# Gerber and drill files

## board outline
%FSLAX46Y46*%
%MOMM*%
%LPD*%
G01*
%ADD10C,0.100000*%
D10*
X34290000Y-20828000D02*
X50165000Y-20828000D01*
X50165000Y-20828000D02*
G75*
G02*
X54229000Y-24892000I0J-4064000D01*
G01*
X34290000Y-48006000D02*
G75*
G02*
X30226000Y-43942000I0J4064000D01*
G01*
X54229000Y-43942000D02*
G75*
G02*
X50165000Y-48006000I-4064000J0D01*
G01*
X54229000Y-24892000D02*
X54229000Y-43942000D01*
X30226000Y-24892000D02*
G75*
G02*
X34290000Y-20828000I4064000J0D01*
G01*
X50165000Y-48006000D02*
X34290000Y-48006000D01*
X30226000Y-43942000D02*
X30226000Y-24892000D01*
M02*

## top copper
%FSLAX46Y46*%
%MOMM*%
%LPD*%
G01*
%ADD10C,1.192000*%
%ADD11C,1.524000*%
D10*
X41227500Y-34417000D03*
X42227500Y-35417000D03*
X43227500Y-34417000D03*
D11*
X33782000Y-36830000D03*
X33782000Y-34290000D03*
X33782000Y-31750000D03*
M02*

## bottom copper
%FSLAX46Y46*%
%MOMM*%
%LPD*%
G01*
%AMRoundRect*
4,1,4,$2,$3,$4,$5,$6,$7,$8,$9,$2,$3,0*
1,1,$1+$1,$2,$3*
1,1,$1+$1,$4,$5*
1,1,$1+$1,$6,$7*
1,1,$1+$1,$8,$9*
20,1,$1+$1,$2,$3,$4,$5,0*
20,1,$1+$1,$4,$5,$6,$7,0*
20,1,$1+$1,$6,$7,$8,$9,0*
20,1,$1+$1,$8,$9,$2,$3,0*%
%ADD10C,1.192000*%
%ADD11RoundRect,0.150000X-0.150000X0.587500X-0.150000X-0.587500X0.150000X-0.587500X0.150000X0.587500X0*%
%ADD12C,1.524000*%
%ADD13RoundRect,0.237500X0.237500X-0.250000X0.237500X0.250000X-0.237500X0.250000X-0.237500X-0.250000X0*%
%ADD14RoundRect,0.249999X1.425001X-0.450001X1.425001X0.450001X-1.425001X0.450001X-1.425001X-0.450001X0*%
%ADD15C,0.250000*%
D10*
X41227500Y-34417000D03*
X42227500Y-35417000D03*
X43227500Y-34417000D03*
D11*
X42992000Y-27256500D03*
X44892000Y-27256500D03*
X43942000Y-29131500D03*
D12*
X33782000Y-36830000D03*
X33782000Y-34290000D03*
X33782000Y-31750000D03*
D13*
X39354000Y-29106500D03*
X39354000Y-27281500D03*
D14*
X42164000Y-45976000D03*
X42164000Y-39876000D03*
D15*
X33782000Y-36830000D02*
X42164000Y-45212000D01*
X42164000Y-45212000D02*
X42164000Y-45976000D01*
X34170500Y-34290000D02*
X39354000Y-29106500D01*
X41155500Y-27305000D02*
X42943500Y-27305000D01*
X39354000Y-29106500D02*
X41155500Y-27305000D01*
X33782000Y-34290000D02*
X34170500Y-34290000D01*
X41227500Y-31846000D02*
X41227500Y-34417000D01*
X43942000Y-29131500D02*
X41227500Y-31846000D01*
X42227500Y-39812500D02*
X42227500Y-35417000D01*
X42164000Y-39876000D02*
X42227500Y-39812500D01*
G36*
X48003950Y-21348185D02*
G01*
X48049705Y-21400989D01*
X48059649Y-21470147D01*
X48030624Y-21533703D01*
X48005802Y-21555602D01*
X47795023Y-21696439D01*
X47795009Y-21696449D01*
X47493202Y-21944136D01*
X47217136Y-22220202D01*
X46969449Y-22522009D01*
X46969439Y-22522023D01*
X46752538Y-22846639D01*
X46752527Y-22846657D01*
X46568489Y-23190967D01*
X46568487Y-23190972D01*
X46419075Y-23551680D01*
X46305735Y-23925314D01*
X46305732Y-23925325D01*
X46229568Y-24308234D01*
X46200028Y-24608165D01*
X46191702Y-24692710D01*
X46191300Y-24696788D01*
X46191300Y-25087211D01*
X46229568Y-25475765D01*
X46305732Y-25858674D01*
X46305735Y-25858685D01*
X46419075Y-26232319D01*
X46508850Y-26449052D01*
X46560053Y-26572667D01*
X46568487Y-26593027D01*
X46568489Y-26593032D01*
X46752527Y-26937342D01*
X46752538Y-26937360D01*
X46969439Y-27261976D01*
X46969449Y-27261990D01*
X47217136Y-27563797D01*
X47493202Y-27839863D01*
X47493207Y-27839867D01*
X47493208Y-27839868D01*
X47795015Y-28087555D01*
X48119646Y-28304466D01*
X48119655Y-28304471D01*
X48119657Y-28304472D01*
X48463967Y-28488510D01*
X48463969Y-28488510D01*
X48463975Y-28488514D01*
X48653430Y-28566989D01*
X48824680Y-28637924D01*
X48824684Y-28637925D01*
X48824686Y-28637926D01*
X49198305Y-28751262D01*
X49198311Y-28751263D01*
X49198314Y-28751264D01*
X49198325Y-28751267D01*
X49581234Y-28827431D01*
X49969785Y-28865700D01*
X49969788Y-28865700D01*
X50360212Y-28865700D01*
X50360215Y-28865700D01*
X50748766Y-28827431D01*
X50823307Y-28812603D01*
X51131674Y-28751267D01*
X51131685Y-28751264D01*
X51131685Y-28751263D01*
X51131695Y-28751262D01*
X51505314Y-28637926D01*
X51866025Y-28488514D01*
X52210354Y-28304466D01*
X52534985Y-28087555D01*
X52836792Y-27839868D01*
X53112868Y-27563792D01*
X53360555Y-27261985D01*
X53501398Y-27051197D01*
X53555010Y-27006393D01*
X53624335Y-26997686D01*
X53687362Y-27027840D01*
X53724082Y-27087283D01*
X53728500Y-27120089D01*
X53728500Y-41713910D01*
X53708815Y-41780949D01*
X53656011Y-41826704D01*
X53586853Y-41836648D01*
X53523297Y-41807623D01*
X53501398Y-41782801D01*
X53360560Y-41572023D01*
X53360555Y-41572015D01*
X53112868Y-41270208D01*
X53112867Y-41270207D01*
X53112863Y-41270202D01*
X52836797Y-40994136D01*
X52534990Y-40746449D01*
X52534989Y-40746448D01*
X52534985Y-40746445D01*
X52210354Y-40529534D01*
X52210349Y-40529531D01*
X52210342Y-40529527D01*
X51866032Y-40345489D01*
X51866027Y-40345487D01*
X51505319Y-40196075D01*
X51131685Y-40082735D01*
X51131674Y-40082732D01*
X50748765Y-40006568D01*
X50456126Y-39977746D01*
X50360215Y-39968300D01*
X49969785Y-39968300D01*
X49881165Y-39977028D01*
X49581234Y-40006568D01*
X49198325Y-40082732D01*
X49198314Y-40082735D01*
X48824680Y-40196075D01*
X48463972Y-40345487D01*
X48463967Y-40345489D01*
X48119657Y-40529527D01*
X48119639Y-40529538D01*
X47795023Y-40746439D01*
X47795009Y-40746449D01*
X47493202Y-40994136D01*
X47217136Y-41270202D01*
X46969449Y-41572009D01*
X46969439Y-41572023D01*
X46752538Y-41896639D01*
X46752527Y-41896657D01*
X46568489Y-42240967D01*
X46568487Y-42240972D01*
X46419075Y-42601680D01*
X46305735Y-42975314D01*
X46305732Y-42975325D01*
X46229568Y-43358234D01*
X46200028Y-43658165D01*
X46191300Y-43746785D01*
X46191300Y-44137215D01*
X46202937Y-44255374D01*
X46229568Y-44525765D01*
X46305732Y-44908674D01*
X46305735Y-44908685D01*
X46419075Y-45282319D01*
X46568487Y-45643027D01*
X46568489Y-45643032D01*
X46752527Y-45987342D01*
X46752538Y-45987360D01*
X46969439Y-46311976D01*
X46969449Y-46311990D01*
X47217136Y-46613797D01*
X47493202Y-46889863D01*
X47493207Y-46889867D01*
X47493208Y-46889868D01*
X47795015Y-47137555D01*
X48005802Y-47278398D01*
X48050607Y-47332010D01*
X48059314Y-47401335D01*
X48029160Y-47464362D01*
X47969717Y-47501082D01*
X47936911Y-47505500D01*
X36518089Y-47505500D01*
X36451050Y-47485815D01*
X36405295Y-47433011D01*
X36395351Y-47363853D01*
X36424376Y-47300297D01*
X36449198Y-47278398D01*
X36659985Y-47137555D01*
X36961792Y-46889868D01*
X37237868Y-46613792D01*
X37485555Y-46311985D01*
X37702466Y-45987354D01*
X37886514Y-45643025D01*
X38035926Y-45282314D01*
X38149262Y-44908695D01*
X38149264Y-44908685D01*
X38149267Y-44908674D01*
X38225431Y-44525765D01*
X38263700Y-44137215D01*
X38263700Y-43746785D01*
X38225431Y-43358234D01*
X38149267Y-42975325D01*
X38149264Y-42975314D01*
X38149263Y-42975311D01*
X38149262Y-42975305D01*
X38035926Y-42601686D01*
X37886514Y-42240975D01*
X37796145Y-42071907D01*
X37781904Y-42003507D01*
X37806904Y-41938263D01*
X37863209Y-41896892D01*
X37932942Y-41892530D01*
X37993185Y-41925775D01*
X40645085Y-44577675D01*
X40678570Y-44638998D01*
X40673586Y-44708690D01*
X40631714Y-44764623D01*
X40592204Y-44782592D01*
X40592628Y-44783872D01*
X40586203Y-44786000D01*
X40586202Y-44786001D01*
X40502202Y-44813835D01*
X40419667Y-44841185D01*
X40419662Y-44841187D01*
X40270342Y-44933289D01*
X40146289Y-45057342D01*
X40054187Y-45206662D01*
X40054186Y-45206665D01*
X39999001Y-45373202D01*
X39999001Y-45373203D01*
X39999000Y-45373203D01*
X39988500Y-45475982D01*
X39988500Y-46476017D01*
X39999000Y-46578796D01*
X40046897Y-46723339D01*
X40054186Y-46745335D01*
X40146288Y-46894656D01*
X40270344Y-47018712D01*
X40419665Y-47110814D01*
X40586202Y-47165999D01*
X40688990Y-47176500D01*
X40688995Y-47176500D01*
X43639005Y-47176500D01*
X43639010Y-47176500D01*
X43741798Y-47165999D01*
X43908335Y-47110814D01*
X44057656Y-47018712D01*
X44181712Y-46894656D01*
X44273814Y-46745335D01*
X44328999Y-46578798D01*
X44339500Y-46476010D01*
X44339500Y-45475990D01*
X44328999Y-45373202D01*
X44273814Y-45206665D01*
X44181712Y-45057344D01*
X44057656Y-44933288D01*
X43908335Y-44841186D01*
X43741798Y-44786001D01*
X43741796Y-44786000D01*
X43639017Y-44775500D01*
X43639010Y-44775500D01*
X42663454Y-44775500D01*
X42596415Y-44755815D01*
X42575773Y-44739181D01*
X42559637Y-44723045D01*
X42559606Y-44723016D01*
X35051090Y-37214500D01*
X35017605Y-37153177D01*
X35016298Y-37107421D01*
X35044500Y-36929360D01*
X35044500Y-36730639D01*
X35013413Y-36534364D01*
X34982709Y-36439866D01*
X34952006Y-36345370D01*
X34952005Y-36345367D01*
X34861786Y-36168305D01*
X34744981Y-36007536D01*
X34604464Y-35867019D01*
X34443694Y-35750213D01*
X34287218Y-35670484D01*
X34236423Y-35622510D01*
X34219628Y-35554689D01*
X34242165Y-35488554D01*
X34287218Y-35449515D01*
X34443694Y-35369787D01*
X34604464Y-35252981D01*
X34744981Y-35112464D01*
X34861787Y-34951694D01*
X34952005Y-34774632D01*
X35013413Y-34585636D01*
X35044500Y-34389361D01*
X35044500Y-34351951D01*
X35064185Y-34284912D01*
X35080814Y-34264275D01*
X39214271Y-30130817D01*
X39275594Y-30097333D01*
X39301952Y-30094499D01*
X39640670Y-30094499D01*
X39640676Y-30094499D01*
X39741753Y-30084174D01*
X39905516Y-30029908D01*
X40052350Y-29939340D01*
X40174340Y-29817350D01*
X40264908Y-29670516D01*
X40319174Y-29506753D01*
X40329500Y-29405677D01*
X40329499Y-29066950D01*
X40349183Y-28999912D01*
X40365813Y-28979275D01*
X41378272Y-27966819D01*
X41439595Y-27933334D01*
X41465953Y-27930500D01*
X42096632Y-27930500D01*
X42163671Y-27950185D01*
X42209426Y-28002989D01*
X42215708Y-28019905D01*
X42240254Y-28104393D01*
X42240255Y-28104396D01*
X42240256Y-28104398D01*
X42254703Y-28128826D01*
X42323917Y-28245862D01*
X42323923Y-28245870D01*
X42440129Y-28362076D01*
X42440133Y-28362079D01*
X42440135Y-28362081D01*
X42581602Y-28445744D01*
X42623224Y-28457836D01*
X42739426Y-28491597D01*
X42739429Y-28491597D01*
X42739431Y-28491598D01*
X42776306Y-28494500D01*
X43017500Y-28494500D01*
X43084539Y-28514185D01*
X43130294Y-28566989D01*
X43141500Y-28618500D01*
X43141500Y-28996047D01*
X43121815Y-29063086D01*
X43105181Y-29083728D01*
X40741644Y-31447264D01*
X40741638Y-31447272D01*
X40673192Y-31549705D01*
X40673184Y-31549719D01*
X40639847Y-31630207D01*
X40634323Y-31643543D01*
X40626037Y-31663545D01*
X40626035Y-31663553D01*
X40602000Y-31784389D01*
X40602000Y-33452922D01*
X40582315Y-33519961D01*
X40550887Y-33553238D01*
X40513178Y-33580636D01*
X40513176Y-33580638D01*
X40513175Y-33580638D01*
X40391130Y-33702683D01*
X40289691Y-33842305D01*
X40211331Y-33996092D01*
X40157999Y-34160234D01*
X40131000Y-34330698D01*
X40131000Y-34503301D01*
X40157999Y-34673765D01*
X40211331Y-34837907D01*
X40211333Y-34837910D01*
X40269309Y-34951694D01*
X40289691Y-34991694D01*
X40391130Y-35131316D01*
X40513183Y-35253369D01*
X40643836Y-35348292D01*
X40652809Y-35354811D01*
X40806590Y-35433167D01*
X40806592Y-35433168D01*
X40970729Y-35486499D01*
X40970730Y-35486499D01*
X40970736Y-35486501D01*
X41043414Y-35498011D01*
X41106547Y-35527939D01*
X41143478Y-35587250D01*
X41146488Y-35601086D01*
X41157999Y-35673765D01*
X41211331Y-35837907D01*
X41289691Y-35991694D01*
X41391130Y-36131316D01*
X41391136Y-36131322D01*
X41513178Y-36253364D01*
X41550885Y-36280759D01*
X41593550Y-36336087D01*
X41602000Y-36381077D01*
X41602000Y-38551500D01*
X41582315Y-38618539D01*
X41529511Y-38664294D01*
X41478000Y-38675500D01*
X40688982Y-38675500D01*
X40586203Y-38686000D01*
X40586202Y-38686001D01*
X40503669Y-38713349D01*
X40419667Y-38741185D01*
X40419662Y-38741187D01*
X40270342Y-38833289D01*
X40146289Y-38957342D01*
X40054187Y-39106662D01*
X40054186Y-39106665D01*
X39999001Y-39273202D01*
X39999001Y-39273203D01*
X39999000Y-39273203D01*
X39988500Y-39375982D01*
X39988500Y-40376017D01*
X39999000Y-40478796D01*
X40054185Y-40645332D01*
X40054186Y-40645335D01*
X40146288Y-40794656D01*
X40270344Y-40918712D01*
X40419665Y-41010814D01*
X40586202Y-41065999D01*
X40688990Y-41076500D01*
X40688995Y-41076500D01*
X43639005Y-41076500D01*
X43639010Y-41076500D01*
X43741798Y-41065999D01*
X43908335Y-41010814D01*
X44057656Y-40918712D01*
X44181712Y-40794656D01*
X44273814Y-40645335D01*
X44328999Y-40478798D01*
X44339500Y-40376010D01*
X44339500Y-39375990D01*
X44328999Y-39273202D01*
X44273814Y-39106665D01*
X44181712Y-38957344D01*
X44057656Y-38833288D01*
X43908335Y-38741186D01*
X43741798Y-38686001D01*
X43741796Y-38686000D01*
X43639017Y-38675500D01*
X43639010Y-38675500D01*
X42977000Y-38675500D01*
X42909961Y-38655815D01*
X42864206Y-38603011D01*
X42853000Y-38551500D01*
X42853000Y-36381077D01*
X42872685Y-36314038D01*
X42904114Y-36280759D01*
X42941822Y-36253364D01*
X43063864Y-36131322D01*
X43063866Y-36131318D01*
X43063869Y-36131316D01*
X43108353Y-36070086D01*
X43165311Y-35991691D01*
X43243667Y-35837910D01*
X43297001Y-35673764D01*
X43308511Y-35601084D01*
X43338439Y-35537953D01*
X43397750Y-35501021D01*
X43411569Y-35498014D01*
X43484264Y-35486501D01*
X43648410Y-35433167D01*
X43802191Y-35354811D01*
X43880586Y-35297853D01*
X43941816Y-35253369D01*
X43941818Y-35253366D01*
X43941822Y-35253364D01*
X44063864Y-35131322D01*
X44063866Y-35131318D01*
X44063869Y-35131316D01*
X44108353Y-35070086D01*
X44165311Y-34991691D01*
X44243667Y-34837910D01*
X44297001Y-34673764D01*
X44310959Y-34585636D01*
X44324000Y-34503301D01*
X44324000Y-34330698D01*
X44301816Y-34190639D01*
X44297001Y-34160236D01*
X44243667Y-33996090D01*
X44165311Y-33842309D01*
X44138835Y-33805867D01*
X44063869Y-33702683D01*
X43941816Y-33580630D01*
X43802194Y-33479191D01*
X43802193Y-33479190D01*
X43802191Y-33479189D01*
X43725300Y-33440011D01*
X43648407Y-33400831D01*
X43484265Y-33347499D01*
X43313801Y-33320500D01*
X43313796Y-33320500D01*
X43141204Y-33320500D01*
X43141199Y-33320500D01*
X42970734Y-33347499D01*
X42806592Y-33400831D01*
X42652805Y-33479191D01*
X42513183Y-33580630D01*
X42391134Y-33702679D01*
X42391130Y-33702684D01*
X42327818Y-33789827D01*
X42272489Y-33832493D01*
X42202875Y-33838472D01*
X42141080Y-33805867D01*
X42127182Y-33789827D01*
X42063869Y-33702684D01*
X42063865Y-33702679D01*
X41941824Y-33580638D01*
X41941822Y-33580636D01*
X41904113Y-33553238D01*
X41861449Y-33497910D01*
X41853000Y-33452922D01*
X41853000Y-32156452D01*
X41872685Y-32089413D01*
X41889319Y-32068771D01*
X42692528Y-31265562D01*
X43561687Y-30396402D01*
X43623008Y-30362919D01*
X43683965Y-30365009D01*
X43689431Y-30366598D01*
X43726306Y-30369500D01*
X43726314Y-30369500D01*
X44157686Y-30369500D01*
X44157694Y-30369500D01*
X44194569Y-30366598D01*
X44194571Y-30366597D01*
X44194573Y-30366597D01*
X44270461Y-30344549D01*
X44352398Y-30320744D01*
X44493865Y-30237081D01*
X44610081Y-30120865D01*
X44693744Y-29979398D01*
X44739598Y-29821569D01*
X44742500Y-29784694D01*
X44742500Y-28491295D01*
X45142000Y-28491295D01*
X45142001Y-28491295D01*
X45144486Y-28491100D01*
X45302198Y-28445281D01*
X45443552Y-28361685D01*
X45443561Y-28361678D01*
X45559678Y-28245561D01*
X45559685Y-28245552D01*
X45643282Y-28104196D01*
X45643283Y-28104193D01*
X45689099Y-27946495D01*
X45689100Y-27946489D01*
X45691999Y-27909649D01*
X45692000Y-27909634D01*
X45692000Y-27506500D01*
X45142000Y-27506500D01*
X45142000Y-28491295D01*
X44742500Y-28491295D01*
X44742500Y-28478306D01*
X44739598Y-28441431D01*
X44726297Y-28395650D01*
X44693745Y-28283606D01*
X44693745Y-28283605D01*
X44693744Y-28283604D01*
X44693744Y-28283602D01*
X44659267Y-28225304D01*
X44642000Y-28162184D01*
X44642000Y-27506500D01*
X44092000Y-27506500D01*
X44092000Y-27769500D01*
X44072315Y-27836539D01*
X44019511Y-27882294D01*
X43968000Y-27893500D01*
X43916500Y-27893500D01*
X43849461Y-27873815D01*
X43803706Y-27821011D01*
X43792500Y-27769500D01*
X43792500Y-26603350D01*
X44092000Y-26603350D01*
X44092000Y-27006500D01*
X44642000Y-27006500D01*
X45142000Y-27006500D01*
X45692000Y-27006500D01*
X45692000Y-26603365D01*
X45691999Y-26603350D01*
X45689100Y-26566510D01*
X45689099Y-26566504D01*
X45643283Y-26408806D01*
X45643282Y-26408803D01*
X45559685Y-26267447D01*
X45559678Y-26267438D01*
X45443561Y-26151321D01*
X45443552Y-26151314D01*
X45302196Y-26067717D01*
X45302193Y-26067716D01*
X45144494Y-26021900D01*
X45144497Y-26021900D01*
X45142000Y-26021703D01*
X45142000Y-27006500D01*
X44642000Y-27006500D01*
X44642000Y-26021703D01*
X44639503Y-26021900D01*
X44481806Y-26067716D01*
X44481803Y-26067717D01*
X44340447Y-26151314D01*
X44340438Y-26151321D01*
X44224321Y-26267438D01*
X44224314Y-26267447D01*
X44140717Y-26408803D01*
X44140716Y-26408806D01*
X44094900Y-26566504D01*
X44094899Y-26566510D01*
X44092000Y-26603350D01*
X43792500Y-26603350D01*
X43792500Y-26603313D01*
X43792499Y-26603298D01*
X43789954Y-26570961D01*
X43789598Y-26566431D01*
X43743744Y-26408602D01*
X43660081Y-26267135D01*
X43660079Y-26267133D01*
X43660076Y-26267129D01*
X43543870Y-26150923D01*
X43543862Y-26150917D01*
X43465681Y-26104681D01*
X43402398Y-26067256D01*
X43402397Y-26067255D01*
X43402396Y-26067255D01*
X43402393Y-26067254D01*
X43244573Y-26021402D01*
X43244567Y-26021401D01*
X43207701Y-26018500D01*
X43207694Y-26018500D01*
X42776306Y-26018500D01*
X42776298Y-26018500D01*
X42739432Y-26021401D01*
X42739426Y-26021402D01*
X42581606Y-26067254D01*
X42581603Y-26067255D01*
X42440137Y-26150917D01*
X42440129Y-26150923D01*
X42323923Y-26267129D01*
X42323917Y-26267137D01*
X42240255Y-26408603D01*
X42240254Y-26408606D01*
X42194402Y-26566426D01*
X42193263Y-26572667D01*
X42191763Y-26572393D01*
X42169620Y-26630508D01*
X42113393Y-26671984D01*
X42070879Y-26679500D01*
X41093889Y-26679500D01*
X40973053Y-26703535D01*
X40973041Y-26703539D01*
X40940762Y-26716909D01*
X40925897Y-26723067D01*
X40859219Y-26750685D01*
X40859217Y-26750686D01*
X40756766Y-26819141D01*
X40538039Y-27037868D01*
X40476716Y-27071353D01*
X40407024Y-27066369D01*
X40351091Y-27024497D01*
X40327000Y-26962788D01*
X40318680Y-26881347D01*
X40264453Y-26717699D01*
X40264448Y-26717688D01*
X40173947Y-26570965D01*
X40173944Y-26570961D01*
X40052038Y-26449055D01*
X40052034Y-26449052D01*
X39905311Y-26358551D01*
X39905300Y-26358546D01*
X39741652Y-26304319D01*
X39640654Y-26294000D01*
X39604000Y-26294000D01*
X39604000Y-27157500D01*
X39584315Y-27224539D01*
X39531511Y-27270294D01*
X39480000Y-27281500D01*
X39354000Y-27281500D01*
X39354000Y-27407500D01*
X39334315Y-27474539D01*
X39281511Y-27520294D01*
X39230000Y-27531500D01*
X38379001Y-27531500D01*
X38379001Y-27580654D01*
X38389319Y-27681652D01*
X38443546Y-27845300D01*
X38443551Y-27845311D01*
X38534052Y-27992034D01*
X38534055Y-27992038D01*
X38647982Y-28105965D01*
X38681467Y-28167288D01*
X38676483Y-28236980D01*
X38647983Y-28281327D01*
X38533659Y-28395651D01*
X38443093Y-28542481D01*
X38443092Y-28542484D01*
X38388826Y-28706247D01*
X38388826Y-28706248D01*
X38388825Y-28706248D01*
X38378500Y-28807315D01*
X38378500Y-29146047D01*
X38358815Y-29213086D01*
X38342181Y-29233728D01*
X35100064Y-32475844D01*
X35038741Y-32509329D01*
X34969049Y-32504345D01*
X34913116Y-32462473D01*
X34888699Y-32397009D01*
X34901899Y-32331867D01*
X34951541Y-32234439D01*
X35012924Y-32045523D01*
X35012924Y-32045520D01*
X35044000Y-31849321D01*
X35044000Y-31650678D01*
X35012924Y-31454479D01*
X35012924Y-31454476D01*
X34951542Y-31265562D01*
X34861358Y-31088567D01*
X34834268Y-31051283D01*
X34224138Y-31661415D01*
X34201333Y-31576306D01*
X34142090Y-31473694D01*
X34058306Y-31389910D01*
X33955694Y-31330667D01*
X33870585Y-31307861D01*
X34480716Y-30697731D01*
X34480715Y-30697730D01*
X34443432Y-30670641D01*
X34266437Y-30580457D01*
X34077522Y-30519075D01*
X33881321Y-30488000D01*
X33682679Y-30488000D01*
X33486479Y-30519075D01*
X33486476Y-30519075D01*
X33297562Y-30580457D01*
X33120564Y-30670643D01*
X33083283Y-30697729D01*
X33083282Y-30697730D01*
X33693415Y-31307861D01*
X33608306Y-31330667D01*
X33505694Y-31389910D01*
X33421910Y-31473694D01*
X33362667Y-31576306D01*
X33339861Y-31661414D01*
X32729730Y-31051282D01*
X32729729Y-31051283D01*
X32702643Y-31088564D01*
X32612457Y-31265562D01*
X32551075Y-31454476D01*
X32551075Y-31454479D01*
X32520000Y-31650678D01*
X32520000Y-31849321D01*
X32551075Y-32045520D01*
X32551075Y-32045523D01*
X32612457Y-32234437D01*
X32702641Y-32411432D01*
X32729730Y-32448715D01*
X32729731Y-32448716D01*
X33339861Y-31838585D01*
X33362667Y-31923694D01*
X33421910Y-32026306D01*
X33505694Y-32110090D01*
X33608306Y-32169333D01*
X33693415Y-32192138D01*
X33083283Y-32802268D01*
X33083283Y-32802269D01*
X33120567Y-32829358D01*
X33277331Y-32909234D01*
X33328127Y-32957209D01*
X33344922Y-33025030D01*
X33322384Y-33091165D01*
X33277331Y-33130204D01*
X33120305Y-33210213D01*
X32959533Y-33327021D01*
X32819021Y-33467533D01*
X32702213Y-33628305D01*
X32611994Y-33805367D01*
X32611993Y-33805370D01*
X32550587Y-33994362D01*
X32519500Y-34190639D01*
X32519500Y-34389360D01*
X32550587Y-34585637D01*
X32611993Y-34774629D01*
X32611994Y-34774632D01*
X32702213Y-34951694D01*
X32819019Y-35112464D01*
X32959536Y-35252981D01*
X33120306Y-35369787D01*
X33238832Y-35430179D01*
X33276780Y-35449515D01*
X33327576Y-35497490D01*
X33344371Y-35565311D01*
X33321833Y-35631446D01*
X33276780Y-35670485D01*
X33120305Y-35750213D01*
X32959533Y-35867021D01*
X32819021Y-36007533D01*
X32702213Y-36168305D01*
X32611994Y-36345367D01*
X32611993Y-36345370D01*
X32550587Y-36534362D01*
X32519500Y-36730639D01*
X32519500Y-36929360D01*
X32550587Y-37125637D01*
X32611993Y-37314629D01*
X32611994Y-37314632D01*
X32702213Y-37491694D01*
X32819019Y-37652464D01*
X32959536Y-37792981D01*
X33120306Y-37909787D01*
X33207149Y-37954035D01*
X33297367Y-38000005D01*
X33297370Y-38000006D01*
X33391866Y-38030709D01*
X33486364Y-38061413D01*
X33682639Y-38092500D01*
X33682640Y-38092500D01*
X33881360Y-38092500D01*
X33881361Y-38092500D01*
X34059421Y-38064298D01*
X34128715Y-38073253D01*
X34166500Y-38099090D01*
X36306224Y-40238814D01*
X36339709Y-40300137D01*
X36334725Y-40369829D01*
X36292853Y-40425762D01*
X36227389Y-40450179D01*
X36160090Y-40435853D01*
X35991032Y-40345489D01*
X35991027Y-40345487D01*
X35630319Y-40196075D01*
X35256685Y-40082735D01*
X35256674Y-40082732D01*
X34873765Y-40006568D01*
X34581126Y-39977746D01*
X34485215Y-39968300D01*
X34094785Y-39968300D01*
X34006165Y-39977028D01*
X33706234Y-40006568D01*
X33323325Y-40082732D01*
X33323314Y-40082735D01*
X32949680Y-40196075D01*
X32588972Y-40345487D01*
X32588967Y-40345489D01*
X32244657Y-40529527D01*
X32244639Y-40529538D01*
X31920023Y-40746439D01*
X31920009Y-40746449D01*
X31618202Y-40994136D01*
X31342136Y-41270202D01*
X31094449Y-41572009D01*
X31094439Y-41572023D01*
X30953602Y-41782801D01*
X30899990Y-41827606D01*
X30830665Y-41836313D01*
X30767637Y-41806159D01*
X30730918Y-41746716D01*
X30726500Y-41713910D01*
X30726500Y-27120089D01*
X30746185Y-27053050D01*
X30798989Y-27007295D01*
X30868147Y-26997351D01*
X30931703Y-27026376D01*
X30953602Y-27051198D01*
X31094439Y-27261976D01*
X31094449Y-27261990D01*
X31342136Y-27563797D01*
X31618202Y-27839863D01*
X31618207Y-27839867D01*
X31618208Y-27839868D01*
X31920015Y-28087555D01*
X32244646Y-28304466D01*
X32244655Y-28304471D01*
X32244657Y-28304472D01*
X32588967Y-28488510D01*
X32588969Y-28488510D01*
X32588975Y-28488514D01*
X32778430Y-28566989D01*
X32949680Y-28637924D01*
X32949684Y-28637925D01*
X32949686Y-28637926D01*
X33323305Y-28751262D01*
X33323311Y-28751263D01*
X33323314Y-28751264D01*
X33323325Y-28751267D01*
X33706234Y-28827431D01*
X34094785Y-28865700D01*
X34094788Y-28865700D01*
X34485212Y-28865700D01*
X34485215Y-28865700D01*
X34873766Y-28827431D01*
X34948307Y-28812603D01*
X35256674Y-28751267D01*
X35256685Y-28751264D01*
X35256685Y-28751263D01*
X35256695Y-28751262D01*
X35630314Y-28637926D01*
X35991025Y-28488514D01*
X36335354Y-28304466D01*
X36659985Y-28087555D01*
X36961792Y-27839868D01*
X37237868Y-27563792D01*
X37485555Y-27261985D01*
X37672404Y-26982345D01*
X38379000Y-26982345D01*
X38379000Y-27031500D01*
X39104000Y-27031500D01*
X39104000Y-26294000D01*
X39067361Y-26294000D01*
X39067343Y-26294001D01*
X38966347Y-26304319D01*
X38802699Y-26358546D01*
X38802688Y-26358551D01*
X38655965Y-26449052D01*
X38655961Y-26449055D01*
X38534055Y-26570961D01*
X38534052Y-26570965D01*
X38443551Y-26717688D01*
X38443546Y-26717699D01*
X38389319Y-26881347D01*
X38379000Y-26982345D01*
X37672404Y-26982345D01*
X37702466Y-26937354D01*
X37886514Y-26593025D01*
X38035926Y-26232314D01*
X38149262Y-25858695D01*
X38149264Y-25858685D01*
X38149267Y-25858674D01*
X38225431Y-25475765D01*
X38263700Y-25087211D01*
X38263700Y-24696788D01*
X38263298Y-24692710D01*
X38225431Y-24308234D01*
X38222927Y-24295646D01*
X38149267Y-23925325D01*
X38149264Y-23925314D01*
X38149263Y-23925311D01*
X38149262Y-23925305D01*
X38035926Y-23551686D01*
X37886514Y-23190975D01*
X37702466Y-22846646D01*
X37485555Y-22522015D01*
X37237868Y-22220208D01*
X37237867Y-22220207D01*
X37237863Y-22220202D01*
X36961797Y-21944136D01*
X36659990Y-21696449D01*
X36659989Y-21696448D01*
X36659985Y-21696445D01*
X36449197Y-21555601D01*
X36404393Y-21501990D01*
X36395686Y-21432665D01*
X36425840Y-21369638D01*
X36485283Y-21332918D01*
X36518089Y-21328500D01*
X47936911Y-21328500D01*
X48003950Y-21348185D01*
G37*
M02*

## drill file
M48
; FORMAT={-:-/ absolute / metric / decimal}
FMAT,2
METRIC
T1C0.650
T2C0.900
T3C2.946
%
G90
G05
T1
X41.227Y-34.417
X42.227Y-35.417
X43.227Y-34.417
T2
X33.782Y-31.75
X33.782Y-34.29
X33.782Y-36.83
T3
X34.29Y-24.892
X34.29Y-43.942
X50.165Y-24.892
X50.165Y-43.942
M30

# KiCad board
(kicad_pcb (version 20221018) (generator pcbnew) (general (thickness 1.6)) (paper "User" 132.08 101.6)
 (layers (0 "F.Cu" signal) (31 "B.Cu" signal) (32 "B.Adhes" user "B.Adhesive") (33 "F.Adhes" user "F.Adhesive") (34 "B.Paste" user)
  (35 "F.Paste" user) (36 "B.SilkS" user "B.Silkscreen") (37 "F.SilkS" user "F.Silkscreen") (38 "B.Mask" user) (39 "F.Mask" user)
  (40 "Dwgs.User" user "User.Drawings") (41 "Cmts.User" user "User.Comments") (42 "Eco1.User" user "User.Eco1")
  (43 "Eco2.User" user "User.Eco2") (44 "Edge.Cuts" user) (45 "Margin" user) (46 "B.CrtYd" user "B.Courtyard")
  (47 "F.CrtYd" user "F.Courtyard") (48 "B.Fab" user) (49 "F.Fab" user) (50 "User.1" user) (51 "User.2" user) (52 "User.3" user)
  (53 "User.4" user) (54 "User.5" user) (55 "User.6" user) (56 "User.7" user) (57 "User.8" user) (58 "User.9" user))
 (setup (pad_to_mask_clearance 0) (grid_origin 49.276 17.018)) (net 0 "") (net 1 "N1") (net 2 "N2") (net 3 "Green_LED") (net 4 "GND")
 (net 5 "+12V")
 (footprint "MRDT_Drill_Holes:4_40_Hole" (layer "F.Cu") (at 50.165 43.942) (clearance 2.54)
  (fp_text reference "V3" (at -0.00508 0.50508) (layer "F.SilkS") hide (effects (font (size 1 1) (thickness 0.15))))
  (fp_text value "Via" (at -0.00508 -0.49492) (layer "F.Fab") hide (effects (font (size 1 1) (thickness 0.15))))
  (pad "" np_thru_hole circle (at 0 0) (size 2.9464 2.9464) (drill 2.9464) (layers "*.Cu" "*.Mask") (clearance 2.5)))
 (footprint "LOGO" (layer "F.Cu") (at 41.91 41.656 90)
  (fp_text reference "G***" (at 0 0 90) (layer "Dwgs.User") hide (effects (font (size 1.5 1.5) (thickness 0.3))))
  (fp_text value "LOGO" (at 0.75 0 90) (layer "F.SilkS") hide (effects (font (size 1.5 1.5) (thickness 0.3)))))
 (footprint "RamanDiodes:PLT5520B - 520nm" (layer "F.Cu") (at 41.2275 34.417)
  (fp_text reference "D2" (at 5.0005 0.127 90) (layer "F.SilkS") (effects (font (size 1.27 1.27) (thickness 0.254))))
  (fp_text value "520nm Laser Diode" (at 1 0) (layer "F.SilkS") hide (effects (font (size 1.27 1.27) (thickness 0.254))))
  (pad "1" thru_hole circle (at 0 0) (size 1.192 1.192) (drill 0.65) (layers "*.Cu" "*.Mask") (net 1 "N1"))
  (pad "2" thru_hole circle (at 1 1) (size 1.192 1.192) (drill 0.65) (layers "*.Cu" "*.Mask") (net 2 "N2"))
  (pad "3" thru_hole circle (at 2 0) (size 1.192 1.192) (drill 0.65) (layers "*.Cu" "*.Mask")))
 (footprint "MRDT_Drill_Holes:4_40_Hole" (layer "F.Cu") (at 34.29 24.892) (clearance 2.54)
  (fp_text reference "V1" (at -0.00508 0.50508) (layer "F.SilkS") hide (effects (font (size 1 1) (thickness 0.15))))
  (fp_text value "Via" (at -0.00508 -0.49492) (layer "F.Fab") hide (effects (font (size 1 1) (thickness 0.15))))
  (pad "" np_thru_hole circle (at 0 0) (size 2.9464 2.9464) (drill 2.9464) (layers "*.Cu" "*.Mask") (clearance 2.5)))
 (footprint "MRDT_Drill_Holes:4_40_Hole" (layer "F.Cu") (at 34.29 43.942) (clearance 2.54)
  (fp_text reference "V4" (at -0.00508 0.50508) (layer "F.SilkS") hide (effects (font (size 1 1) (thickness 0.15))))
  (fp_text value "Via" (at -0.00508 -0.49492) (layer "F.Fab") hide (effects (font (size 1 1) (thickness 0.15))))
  (pad "" np_thru_hole circle (at 0 0) (size 2.9464 2.9464) (drill 2.9464) (layers "*.Cu" "*.Mask") (clearance 2.5)))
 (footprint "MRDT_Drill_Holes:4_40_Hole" (layer "F.Cu") (at 50.165 24.892) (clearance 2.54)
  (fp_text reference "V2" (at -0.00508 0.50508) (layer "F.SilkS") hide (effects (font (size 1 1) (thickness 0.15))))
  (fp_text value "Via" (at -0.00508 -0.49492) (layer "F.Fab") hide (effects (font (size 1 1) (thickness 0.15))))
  (pad "" np_thru_hole circle (at 0 0) (size 2.9464 2.9464) (drill 2.9464) (layers "*.Cu" "*.Mask") (clearance 2.5)))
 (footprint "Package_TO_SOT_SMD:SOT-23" (layer "B.Cu") (at 43.942 28.194 -90)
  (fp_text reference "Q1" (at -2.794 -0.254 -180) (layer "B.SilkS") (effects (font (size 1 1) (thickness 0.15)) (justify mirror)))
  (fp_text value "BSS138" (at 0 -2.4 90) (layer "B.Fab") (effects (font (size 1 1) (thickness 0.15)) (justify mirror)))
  (pad "1" smd roundrect (at -0.9375 0.95 270) (size 1.475 0.6) (layers "B.Cu" "B.Paste" "B.Mask") (roundrect_rratio 0.25)
   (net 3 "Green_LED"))
  (pad "2" smd roundrect (at -0.9375 -0.95 270) (size 1.475 0.6) (layers "B.Cu" "B.Paste" "B.Mask") (roundrect_rratio 0.25) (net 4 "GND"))
  (pad "3" smd roundrect (at 0.9375 0 270) (size 1.475 0.6) (layers "B.Cu" "B.Paste" "B.Mask") (roundrect_rratio 0.25) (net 1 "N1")))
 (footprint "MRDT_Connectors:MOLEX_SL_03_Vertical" (layer "B.Cu") (at 33.782 36.83 90)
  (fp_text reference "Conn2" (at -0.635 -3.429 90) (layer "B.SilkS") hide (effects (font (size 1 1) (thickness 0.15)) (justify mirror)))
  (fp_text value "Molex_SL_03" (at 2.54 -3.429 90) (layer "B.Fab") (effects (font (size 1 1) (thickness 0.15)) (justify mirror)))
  (pad "1" thru_hole circle (at 0 0 90) (size 1.524 1.524) (drill 0.9) (layers "*.Cu" "*.Mask") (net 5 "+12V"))
  (pad "2" thru_hole circle (at 2.54 0 90) (size 1.524 1.524) (drill 0.9) (layers "*.Cu" "*.Mask") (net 3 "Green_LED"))
  (pad "3" thru_hole circle (at 5.08 0 90) (size 1.524 1.524) (drill 0.9) (layers "*.Cu" "*.Mask") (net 4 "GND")))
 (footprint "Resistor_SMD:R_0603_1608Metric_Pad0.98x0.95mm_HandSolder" (layer "B.Cu") (at 39.354 28.194 90)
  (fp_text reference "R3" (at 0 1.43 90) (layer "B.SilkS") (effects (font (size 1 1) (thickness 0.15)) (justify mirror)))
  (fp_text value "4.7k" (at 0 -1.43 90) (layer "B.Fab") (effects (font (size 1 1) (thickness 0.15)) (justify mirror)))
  (pad "1" smd roundrect (at -0.9125 0 90) (size 0.975 0.95) (layers "B.Cu" "B.Paste" "B.Mask") (roundrect_rratio 0.25) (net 3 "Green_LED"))
  (pad "2" smd roundrect (at 0.9125 0 90) (size 0.975 0.95) (layers "B.Cu" "B.Paste" "B.Mask") (roundrect_rratio 0.25) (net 4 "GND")))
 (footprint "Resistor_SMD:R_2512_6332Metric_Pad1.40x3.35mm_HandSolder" (layer "B.Cu") (at 42.164 42.926 90)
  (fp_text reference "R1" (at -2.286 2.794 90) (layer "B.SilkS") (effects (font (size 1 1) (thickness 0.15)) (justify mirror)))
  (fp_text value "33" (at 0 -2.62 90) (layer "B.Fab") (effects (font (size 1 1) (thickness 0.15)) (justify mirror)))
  (pad "1" smd roundrect (at -3.05 0 90) (size 1.4 3.35) (layers "B.Cu" "B.Paste" "B.Mask") (roundrect_rratio 0.178571) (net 5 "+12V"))
  (pad "2" smd roundrect (at 3.05 0 90) (size 1.4 3.35) (layers "B.Cu" "B.Paste" "B.Mask") (roundrect_rratio 0.178571) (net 2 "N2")))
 (gr_line (start 34.29 20.828) (end 50.165 20.828) (stroke (width 0.1) (type default)) (layer "Edge.Cuts"))
 (gr_arc (start 50.165 20.828) (mid 53.038682 22.018318) (end 54.229 24.892) (stroke (width 0.1) (type default)) (layer "Edge.Cuts"))
 (gr_arc (start 34.29 48.006) (mid 31.416318 46.815682) (end 30.226 43.942) (stroke (width 0.1) (type default)) (layer "Edge.Cuts"))
 (gr_arc (start 54.229 43.942) (mid 53.038682 46.815682) (end 50.165 48.006) (stroke (width 0.1) (type default)) (layer "Edge.Cuts"))
 (gr_line (start 54.229 24.892) (end 54.229 43.942) (stroke (width 0.1) (type default)) (layer "Edge.Cuts"))
 (gr_arc (start 30.226 24.892) (mid 31.416318 22.018318) (end 34.29 20.828) (stroke (width 0.1) (type default)) (layer "Edge.Cuts"))
 (gr_line (start 50.165 48.006) (end 34.29 48.006) (stroke (width 0.1) (type default)) (layer "Edge.Cuts"))
 (gr_line (start 30.226 43.942) (end 30.226 24.892) (stroke (width 0.1) (type default)) (layer "Edge.Cuts"))
 (segment (start 33.782 36.83) (end 42.164 45.212) (width 0.25) (layer "B.Cu") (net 5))
 (segment (start 42.164 45.212) (end 42.164 45.976) (width 0.25) (layer "B.Cu") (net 5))
 (segment (start 34.1705 34.29) (end 39.354 29.1065) (width 0.25) (layer "B.Cu") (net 3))
 (segment (start 41.1555 27.305) (end 42.9435 27.305) (width 0.25) (layer "B.Cu") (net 3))
 (segment (start 39.354 29.1065) (end 41.1555 27.305) (width 0.25) (layer "B.Cu") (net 3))
 (segment (start 33.782 34.29) (end 34.1705 34.29) (width 0.25) (layer "B.Cu") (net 3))
 (segment (start 41.2275 31.846) (end 41.2275 34.417) (width 0.25) (layer "B.Cu") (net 1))
 (segment (start 43.942 29.1315) (end 41.2275 31.846) (width 0.25) (layer "B.Cu") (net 1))
 (segment (start 42.2275 39.8125) (end 42.2275 35.417) (width 0.25) (layer "B.Cu") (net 2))
 (segment (start 42.164 39.876) (end 42.2275 39.8125) (width 0.25) (layer "B.Cu") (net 2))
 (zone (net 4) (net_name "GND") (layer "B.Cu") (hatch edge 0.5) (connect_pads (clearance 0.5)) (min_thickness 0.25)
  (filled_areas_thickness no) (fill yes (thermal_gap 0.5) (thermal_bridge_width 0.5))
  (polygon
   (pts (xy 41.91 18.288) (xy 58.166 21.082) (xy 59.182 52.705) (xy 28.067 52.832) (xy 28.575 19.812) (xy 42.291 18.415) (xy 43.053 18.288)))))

